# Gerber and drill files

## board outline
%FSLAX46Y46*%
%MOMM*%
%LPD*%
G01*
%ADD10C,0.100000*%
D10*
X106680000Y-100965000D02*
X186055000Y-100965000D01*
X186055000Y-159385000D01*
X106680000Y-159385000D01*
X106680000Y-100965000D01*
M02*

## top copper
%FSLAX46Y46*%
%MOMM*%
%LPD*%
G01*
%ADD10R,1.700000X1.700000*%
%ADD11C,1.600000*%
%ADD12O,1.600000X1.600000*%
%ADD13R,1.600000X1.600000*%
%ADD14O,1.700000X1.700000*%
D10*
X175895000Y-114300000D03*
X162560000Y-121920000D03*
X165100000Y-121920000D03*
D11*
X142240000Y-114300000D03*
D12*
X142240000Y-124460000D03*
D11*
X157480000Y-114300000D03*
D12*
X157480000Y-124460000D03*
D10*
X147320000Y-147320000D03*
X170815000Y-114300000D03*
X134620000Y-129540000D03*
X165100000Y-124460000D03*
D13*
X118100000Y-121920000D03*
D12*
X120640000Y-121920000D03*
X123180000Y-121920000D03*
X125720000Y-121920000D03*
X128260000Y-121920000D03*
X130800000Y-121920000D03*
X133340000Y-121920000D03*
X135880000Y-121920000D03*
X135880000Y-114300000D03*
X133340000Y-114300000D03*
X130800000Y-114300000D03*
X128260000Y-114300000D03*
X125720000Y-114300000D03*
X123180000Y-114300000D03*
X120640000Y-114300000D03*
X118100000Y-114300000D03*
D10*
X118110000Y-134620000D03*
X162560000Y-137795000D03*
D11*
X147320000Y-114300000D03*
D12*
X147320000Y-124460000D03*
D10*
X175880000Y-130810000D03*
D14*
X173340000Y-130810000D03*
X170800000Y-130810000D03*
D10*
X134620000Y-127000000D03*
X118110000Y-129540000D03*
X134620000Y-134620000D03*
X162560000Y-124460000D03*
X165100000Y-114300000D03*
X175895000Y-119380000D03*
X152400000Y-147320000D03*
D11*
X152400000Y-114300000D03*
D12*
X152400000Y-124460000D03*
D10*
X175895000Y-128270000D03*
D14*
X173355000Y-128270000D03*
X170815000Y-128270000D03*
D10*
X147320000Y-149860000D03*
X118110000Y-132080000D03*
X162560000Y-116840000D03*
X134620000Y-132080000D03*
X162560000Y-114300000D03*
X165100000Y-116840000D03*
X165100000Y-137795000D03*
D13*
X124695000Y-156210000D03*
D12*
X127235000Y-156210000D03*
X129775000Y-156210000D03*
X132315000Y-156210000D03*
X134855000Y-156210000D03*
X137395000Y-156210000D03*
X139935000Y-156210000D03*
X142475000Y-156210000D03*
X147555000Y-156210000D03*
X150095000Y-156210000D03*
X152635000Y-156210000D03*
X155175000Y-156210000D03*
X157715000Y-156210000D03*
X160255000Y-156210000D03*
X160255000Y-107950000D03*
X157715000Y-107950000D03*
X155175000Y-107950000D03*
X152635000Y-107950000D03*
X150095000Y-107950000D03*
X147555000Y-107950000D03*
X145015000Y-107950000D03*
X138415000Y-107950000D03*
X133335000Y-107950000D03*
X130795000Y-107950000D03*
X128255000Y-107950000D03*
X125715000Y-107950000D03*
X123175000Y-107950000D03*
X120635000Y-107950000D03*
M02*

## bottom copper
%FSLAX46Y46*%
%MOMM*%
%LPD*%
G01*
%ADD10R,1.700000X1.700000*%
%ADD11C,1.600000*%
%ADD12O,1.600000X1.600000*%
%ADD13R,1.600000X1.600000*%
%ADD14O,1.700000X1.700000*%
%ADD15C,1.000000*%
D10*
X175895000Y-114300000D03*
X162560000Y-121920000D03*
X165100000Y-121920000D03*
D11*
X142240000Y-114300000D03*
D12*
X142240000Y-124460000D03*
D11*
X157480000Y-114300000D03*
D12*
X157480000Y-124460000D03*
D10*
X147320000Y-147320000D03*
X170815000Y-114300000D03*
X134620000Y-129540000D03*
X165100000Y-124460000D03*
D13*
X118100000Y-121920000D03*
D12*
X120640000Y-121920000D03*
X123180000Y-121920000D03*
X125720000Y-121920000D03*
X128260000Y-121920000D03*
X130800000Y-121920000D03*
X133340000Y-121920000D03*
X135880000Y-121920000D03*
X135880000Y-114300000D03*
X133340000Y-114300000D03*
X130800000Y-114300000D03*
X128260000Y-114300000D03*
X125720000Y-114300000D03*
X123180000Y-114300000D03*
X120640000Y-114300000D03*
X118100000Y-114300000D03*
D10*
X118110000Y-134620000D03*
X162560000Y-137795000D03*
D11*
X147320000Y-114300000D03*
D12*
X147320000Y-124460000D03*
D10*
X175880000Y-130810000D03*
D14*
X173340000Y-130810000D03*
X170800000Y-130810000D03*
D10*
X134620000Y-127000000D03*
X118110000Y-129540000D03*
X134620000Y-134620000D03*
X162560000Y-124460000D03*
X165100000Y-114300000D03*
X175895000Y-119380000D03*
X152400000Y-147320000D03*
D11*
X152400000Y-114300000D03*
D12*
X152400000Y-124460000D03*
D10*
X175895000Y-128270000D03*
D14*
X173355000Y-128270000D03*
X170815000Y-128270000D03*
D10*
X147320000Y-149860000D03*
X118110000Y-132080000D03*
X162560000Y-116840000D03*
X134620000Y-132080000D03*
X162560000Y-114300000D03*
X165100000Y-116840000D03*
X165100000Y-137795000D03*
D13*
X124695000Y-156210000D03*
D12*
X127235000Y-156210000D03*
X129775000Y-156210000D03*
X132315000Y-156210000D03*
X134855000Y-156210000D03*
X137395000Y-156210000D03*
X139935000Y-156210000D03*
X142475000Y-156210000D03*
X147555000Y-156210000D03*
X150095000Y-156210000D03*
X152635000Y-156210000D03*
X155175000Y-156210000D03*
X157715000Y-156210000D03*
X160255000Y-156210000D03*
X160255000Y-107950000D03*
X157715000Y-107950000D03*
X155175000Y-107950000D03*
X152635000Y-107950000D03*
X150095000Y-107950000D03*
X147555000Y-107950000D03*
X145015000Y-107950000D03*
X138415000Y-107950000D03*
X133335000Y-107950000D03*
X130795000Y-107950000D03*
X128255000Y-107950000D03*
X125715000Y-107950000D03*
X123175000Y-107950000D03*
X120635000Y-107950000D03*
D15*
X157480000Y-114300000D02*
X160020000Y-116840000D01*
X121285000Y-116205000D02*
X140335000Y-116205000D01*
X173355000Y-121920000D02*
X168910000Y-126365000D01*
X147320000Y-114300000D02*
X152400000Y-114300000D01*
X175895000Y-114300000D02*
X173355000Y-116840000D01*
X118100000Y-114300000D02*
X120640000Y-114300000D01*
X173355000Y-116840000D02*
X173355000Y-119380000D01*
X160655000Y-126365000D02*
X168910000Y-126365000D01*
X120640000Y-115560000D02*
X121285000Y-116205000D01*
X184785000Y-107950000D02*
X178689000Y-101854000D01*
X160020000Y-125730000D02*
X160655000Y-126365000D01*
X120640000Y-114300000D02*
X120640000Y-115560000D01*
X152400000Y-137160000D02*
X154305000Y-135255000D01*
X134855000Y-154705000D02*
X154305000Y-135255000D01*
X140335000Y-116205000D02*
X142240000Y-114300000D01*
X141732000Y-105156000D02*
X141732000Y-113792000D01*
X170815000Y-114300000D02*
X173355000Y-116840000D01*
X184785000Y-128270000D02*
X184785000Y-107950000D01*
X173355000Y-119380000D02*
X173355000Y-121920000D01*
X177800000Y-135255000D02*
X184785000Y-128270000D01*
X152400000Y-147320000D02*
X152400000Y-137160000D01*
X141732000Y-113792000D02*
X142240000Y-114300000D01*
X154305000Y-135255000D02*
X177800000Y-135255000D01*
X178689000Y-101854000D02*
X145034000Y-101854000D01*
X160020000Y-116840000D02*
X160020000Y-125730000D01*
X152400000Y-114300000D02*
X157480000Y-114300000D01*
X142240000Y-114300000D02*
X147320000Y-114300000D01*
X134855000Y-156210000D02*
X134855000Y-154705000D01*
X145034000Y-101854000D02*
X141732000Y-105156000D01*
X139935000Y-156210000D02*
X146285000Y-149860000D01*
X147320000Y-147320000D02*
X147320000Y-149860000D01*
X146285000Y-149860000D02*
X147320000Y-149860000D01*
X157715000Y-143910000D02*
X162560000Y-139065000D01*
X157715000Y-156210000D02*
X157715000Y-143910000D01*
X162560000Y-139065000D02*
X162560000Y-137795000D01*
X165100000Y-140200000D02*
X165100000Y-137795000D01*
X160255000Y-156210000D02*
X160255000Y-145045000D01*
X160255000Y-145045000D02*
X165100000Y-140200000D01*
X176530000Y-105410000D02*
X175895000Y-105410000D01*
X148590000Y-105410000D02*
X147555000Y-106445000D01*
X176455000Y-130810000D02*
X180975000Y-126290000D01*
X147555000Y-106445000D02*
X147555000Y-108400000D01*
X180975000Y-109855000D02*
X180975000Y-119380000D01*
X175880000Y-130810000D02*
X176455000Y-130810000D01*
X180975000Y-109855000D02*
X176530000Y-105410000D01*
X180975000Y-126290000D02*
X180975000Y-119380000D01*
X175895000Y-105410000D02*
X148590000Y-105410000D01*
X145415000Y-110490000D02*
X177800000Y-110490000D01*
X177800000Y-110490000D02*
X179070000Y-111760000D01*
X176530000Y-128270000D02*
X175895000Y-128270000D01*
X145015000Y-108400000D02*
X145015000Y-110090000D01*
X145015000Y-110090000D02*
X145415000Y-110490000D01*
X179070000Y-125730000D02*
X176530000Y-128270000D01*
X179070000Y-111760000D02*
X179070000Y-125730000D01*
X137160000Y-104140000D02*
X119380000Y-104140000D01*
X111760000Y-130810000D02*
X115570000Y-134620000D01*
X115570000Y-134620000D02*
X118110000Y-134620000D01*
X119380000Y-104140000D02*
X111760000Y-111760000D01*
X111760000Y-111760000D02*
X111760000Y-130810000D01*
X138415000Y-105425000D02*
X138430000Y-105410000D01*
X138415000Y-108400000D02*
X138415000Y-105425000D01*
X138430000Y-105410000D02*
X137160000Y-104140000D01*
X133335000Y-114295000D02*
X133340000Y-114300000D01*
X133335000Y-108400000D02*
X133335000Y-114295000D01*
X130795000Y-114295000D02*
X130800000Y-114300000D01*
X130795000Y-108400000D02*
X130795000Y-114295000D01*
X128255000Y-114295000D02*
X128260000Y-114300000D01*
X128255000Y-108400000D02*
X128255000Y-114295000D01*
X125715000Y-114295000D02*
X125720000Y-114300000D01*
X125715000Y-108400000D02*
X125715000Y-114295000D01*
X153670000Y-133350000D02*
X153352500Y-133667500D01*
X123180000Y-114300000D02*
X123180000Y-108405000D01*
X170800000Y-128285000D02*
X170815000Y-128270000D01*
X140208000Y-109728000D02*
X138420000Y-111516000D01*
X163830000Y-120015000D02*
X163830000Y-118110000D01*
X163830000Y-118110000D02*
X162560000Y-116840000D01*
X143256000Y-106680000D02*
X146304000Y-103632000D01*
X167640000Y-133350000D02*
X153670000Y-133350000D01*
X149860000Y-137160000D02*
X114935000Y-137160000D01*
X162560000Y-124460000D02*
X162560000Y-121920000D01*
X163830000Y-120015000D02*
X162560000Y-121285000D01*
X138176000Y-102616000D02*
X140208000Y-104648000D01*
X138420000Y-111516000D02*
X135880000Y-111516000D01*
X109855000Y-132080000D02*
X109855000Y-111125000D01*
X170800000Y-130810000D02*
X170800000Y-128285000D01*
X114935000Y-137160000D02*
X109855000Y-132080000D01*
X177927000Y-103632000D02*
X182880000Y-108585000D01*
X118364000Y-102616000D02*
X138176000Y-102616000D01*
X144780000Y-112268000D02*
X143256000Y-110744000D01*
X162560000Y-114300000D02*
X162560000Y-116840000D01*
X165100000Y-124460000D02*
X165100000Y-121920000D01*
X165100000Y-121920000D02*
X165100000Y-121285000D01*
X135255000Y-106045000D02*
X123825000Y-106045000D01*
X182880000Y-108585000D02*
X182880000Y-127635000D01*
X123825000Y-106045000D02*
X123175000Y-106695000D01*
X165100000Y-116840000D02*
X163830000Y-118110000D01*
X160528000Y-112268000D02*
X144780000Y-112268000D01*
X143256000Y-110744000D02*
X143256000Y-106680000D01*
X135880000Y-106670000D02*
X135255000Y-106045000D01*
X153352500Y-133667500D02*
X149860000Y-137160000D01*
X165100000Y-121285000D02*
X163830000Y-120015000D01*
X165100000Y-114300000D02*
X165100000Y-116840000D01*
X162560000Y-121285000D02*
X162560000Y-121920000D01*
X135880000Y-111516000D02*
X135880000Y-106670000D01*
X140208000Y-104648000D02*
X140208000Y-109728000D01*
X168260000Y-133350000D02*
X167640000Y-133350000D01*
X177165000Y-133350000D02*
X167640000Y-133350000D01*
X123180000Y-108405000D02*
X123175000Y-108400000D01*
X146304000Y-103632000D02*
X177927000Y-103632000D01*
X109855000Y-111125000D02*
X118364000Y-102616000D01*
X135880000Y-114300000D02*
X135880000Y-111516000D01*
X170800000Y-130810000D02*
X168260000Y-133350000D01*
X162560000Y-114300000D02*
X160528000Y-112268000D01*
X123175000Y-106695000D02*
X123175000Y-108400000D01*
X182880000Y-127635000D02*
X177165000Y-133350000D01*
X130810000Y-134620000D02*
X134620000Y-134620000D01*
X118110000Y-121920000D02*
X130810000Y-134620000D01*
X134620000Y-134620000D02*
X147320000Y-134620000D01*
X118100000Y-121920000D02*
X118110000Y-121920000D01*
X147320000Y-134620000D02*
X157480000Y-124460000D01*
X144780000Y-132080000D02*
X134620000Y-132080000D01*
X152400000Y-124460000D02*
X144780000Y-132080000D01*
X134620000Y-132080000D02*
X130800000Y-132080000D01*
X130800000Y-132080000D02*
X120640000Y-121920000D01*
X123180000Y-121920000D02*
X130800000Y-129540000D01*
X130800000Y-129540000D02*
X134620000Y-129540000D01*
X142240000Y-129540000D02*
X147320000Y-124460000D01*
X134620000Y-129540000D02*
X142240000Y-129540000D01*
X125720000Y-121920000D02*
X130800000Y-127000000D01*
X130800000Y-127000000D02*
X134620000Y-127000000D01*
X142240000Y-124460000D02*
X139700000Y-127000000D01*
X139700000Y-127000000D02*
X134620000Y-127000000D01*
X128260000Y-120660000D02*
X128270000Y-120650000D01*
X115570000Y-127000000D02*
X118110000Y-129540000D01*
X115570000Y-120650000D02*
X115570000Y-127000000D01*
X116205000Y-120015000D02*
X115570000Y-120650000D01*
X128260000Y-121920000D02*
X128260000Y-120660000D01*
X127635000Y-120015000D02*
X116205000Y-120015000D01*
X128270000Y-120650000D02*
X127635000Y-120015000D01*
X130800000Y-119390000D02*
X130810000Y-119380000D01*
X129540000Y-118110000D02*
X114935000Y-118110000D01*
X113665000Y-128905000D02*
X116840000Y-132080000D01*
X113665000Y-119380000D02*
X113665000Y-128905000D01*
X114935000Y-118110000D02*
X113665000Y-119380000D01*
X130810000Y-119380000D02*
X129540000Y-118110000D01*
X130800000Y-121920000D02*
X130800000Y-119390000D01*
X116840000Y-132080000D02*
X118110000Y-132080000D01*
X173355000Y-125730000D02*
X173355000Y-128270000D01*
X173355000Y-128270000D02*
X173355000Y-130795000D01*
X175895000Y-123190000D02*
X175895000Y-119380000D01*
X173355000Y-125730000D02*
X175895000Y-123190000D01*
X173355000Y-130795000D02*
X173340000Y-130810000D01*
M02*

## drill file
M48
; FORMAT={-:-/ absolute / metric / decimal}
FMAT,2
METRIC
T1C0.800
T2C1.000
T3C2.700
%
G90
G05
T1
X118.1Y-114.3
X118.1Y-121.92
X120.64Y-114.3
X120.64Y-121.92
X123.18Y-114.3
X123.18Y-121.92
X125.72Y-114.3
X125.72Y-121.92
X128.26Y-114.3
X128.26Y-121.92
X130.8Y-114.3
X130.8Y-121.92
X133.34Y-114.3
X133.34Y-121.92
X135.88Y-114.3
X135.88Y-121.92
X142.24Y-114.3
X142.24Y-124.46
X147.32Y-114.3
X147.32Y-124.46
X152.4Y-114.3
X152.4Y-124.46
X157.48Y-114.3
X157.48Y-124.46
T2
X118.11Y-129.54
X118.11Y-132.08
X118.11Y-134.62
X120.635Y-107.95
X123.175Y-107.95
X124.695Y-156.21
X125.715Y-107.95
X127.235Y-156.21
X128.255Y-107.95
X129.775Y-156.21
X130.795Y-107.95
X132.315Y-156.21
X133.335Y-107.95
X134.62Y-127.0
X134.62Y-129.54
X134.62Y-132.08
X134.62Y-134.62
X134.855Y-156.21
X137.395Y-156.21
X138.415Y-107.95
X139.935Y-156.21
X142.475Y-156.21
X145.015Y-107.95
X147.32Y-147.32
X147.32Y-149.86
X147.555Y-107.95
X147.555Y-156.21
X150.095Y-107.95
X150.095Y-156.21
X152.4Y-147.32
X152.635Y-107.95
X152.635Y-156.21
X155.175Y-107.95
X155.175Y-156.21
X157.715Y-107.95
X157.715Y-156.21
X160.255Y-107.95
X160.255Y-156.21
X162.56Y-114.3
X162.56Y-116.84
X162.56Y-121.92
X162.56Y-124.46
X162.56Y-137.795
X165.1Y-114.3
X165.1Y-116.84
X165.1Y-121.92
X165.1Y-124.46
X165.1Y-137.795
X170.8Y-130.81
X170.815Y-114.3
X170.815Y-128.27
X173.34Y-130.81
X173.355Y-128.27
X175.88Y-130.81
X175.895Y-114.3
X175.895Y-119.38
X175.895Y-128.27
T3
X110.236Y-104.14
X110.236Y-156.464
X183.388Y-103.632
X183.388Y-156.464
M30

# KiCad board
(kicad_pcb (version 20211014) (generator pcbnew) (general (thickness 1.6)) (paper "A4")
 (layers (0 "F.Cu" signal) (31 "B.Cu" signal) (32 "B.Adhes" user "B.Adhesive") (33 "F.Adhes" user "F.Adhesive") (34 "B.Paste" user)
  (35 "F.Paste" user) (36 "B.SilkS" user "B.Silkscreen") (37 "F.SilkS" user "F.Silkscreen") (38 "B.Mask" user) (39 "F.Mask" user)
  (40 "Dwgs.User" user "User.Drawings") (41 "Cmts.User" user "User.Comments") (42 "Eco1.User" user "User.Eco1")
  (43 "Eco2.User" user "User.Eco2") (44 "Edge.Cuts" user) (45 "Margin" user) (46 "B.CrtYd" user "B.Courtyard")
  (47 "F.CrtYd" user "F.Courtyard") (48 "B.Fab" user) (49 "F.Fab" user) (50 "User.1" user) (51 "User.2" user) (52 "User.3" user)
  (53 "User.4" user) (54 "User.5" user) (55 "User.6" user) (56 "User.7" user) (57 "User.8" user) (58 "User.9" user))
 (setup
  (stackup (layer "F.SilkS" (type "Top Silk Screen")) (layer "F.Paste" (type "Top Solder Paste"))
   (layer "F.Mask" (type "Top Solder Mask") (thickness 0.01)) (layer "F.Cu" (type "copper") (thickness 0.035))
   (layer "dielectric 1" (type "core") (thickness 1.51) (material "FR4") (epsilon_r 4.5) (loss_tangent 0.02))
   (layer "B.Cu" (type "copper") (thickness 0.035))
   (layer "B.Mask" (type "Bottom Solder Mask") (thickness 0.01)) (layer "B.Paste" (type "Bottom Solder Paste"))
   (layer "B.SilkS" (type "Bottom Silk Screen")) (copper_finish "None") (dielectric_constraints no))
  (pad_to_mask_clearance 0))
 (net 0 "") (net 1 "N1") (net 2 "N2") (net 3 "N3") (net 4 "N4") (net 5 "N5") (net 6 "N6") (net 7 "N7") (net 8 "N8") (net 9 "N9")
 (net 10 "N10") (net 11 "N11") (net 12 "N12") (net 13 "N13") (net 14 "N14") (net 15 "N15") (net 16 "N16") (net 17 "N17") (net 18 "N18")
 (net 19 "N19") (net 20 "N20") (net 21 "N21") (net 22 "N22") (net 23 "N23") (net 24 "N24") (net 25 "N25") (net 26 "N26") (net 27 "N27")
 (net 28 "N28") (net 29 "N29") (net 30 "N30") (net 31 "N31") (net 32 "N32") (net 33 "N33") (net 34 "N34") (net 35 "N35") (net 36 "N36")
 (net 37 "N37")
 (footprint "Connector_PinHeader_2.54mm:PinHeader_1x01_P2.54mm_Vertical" (layer "F.Cu") (at 175.895 114.3)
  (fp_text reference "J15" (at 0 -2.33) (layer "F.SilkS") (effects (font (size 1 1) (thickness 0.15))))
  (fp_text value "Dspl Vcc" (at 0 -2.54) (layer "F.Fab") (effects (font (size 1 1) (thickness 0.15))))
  (pad "1" thru_hole rect (at 0 0) (size 1.7 1.7) (drill 1) (layers *.Cu *.Mask) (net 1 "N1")))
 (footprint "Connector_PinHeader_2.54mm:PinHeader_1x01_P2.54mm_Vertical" (layer "F.Cu") (at 162.56 121.92)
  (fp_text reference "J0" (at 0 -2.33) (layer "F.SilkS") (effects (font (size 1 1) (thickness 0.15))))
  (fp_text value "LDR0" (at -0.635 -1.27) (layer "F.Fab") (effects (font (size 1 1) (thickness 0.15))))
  (pad "1" thru_hole rect (at 0 0) (size 1.7 1.7) (drill 1) (layers *.Cu *.Mask) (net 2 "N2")))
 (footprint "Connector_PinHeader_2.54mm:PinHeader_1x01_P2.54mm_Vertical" (layer "F.Cu") (at 165.1 121.92)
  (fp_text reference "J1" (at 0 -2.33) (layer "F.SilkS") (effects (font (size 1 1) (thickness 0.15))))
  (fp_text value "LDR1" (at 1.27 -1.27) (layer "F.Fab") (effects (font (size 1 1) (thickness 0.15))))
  (pad "1" thru_hole rect (at 0 0) (size 1.7 1.7) (drill 1) (layers *.Cu *.Mask) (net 2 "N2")))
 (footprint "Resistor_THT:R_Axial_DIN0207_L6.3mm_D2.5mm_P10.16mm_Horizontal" (layer "F.Cu") (at 142.24 114.3 -90)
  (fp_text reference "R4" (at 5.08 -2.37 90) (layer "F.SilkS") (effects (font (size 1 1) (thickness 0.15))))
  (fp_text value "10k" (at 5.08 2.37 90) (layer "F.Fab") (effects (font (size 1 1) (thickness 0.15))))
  (pad "1" thru_hole circle (at 0 0 270) (size 1.6 1.6) (drill 0.8) (layers *.Cu *.Mask) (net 1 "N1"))
  (pad "2" thru_hole oval (at 10.16 0 270) (size 1.6 1.6) (drill 0.8) (layers *.Cu *.Mask) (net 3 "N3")))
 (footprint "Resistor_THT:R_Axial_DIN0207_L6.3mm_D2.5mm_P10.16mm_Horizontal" (layer "F.Cu") (at 157.48 114.3 -90)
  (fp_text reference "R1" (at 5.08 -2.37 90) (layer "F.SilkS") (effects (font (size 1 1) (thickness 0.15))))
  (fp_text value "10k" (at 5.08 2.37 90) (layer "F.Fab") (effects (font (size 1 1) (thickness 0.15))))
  (pad "1" thru_hole circle (at 0 0 270) (size 1.6 1.6) (drill 0.8) (layers *.Cu *.Mask) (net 1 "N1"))
  (pad "2" thru_hole oval (at 10.16 0 270) (size 1.6 1.6) (drill 0.8) (layers *.Cu *.Mask) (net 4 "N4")))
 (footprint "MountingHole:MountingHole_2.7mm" (layer "F.Cu") (at 110.236 156.464)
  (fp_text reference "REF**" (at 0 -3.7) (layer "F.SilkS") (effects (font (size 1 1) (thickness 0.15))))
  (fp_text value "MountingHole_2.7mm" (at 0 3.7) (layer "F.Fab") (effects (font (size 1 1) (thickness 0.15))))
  (pad "" np_thru_hole circle (at 0 0) (size 2.7 2.7) (drill 2.7) (layers *.Cu *.Mask)))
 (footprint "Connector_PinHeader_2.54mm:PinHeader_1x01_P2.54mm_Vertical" (layer "F.Cu") (at 147.32 147.32)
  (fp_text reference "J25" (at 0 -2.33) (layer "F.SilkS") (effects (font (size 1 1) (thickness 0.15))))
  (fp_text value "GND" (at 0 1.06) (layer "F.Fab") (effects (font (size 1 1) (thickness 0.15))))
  (pad "1" thru_hole rect (at 0 0) (size 1.7 1.7) (drill 1) (layers *.Cu *.Mask) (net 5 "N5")))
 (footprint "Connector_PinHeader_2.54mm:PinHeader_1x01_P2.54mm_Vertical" (layer "F.Cu") (at 170.815 114.3)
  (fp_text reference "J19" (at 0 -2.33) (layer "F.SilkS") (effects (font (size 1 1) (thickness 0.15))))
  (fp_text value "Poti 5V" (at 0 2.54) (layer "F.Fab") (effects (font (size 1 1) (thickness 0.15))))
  (pad "1" thru_hole rect (at 0 0) (size 1.7 1.7) (drill 1) (layers *.Cu *.Mask) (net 1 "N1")))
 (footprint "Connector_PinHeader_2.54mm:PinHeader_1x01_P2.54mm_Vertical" (layer "F.Cu") (at 134.62 129.54 90)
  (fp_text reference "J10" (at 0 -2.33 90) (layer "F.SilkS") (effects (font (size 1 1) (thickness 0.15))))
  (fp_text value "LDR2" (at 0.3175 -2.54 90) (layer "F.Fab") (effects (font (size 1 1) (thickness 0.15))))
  (pad "1" thru_hole rect (at 0 0 90) (size 1.7 1.7) (drill 1) (layers *.Cu *.Mask) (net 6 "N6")))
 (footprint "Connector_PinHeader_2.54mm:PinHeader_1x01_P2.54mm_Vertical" (layer "F.Cu") (at 165.1 124.46)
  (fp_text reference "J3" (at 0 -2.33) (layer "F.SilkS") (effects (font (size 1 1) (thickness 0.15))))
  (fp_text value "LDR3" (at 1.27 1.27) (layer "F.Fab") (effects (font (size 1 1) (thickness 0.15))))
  (pad "1" thru_hole rect (at 0 0) (size 1.7 1.7) (drill 1) (layers *.Cu *.Mask) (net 2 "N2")))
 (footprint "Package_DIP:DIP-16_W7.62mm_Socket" (layer "F.Cu") (at 118.1 121.92 90)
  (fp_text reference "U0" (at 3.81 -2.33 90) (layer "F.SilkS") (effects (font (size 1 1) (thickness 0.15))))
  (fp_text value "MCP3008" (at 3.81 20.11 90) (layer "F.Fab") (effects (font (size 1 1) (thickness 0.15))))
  (pad "1" thru_hole rect (at 0 0 90) (size 1.6 1.6) (drill 0.8) (layers *.Cu *.Mask) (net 4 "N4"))
  (pad "2" thru_hole oval (at 0 2.54 90) (size 1.6 1.6) (drill 0.8) (layers *.Cu *.Mask) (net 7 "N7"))
  (pad "3" thru_hole oval (at 0 5.08 90) (size 1.6 1.6) (drill 0.8) (layers *.Cu *.Mask) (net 6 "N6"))
  (pad "4" thru_hole oval (at 0 7.62 90) (size 1.6 1.6) (drill 0.8) (layers *.Cu *.Mask) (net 3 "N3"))
  (pad "5" thru_hole oval (at 0 10.16 90) (size 1.6 1.6) (drill 0.8) (layers *.Cu *.Mask) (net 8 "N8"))
  (pad "6" thru_hole oval (at 0 12.7 90) (size 1.6 1.6) (drill 0.8) (layers *.Cu *.Mask) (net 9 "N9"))
  (pad "7" thru_hole oval (at 0 15.24 90) (size 1.6 1.6) (drill 0.8) (layers *.Cu *.Mask) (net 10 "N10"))
  (pad "8" thru_hole oval (at 0 17.78 90) (size 1.6 1.6) (drill 0.8) (layers *.Cu *.Mask) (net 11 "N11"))
  (pad "9" thru_hole oval (at 7.62 17.78 90) (size 1.6 1.6) (drill 0.8) (layers *.Cu *.Mask) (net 2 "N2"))
  (pad "10" thru_hole oval (at 7.62 15.24 90) (size 1.6 1.6) (drill 0.8) (layers *.Cu *.Mask) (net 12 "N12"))
  (pad "11" thru_hole oval (at 7.62 12.7 90) (size 1.6 1.6) (drill 0.8) (layers *.Cu *.Mask) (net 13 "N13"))
  (pad "12" thru_hole oval (at 7.62 10.16 90) (size 1.6 1.6) (drill 0.8) (layers *.Cu *.Mask) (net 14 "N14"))
  (pad "13" thru_hole oval (at 7.62 7.62 90) (size 1.6 1.6) (drill 0.8) (layers *.Cu *.Mask) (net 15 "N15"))
  (pad "14" thru_hole oval (at 7.62 5.08 90) (size 1.6 1.6) (drill 0.8) (layers *.Cu *.Mask) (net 2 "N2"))
  (pad "15" thru_hole oval (at 7.62 2.54 90) (size 1.6 1.6) (drill 0.8) (layers *.Cu *.Mask) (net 1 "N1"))
  (pad "16" thru_hole oval (at 7.62 0 90) (size 1.6 1.6) (drill 0.8) (layers *.Cu *.Mask) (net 1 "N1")))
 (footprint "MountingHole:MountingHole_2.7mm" (layer "F.Cu") (at 183.388 156.464)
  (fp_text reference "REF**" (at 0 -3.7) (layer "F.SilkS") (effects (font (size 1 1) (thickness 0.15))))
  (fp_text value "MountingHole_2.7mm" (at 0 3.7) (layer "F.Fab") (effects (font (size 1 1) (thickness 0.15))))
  (pad "" np_thru_hole circle (at 0 0) (size 2.7 2.7) (drill 2.7) (layers *.Cu *.Mask)))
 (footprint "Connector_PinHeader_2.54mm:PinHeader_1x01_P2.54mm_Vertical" (layer "F.Cu") (at 118.11 134.62 -90)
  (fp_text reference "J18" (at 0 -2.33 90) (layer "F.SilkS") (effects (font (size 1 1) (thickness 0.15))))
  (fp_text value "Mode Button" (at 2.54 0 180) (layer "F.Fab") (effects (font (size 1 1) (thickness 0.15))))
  (pad "1" thru_hole rect (at 0 0 270) (size 1.7 1.7) (drill 1) (layers *.Cu *.Mask) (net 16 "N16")))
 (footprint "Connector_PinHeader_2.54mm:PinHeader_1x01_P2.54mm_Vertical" (layer "F.Cu") (at 162.56 137.795)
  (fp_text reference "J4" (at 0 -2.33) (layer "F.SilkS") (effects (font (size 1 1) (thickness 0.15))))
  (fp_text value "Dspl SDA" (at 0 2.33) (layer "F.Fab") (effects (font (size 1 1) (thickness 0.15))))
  (pad "1" thru_hole rect (at 0 0) (size 1.7 1.7) (drill 1) (layers *.Cu *.Mask) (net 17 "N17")))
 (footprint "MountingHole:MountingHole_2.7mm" (layer "F.Cu") (at 110.236 104.14)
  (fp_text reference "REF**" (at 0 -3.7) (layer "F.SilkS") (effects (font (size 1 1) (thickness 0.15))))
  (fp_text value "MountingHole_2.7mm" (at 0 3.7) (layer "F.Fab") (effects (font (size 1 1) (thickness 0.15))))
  (pad "" np_thru_hole circle (at 0 0) (size 2.7 2.7) (drill 2.7) (layers *.Cu *.Mask)))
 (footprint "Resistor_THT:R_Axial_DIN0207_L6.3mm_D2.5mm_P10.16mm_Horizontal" (layer "F.Cu") (at 147.32 114.3 -90)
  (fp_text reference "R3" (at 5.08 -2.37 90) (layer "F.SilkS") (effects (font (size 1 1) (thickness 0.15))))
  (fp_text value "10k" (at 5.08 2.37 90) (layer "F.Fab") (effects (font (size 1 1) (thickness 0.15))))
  (pad "1" thru_hole circle (at 0 0 270) (size 1.6 1.6) (drill 0.8) (layers *.Cu *.Mask) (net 1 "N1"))
  (pad "2" thru_hole oval (at 10.16 0 270) (size 1.6 1.6) (drill 0.8) (layers *.Cu *.Mask) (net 6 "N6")))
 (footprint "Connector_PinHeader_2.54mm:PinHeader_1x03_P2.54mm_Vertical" (layer "F.Cu") (at 175.88 130.81 -90)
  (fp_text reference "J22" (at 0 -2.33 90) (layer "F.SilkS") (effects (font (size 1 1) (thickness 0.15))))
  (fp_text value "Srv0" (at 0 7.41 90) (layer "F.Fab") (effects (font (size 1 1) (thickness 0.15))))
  (pad "1" thru_hole rect (at 0 0 270) (size 1.7 1.7) (drill 1) (layers *.Cu *.Mask) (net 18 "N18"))
  (pad "2" thru_hole oval (at 0 2.54 270) (size 1.7 1.7) (drill 1) (layers *.Cu *.Mask) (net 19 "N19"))
  (pad "3" thru_hole oval (at 0 5.08 270) (size 1.7 1.7) (drill 1) (layers *.Cu *.Mask) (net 2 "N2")))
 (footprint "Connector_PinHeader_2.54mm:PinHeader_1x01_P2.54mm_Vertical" (layer "F.Cu") (at 134.62 127)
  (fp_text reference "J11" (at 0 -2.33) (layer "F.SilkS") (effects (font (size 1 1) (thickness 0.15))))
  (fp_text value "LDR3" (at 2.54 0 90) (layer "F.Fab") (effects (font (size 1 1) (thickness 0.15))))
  (pad "1" thru_hole rect (at 0 0) (size 1.7 1.7) (drill 1) (layers *.Cu *.Mask) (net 3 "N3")))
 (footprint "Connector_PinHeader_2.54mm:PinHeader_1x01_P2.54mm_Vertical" (layer "F.Cu") (at 118.11 129.54 -90)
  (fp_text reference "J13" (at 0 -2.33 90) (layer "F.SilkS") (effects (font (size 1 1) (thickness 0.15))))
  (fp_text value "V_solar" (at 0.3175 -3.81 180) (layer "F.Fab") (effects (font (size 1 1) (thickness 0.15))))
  (pad "1" thru_hole rect (at 0 0 270) (size 1.7 1.7) (drill 1) (layers *.Cu *.Mask) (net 8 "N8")))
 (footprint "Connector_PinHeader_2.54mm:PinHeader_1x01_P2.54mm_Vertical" (layer "F.Cu") (at 134.62 134.62 90)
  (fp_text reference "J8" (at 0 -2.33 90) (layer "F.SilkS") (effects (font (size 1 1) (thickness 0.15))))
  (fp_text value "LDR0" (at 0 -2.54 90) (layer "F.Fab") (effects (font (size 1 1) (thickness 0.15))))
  (pad "1" thru_hole rect (at 0 0 90) (size 1.7 1.7) (drill 1) (layers *.Cu *.Mask) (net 4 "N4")))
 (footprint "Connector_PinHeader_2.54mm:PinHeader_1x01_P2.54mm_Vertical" (layer "F.Cu") (at 162.56 124.46)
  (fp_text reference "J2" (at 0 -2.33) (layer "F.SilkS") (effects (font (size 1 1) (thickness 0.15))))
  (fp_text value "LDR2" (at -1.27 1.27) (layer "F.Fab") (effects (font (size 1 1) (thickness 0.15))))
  (pad "1" thru_hole rect (at 0 0) (size 1.7 1.7) (drill 1) (layers *.Cu *.Mask) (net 2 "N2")))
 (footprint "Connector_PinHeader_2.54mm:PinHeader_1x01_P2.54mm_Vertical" (layer "F.Cu") (at 165.1 114.3)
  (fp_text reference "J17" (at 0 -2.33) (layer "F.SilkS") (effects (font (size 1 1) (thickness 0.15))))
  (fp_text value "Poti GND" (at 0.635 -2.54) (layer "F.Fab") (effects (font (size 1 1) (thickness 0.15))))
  (pad "1" thru_hole rect (at 0 0) (size 1.7 1.7) (drill 1) (layers *.Cu *.Mask) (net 2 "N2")))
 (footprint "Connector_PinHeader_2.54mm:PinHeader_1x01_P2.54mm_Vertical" (layer "F.Cu") (at 175.895 119.38)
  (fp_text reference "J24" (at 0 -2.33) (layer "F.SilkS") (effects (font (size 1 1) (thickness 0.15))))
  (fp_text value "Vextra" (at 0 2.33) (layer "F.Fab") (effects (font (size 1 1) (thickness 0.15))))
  (pad "1" thru_hole rect (at 0 0) (size 1.7 1.7) (drill 1) (layers *.Cu *.Mask) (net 19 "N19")))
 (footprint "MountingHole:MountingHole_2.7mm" (layer "F.Cu") (at 183.388 103.632)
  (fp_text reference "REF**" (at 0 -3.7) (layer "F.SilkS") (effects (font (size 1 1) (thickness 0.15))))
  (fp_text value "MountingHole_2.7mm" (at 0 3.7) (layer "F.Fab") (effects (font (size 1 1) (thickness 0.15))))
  (pad "" np_thru_hole circle (at 0 0) (size 2.7 2.7) (drill 2.7) (layers *.Cu *.Mask)))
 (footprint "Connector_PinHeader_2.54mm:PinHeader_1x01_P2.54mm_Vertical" (layer "F.Cu") (at 152.4 147.32)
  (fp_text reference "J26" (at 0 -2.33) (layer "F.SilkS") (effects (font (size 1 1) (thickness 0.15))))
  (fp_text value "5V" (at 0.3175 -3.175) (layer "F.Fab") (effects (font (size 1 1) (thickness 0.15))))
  (pad "1" thru_hole rect (at 0 0) (size 1.7 1.7) (drill 1) (layers *.Cu *.Mask) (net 1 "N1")))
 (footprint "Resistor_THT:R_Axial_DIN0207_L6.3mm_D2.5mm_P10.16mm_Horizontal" (layer "F.Cu") (at 152.4 114.3 -90)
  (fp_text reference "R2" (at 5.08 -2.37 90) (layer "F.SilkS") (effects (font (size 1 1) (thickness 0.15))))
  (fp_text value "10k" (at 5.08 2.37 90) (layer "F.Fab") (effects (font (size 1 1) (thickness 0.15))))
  (pad "1" thru_hole circle (at 0 0 270) (size 1.6 1.6) (drill 0.8) (layers *.Cu *.Mask) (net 1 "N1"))
  (pad "2" thru_hole oval (at 10.16 0 270) (size 1.6 1.6) (drill 0.8) (layers *.Cu *.Mask) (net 7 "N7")))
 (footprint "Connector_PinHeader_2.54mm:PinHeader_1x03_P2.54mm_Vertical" (layer "F.Cu") (at 175.895 128.27 -90)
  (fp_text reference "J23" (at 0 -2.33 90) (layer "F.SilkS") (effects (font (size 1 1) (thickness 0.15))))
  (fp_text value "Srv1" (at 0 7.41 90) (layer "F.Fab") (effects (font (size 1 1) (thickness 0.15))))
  (pad "1" thru_hole rect (at 0 0 270) (size 1.7 1.7) (drill 1) (layers *.Cu *.Mask) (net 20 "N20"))
  (pad "2" thru_hole oval (at 0 2.54 270) (size 1.7 1.7) (drill 1) (layers *.Cu *.Mask) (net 19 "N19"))
  (pad "3" thru_hole oval (at 0 5.08 270) (size 1.7 1.7) (drill 1) (layers *.Cu *.Mask) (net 2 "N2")))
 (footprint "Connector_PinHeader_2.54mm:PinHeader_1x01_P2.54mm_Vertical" (layer "F.Cu") (at 147.32 149.86)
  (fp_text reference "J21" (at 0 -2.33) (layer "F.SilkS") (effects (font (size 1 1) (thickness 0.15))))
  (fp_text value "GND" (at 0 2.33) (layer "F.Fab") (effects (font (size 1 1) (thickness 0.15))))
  (pad "1" thru_hole rect (at 0 0) (size 1.7 1.7) (drill 1) (layers *.Cu *.Mask) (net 5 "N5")))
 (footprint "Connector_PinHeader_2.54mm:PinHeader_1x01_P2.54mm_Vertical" (layer "F.Cu") (at 118.11 132.08 -90)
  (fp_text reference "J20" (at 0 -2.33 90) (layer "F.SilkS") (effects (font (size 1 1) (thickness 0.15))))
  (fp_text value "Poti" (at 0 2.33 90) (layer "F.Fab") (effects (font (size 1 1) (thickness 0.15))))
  (pad "1" thru_hole rect (at 0 0 270) (size 1.7 1.7) (drill 1) (layers *.Cu *.Mask) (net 9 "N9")))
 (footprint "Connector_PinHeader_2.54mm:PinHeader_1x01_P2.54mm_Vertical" (layer "F.Cu") (at 162.56 116.84)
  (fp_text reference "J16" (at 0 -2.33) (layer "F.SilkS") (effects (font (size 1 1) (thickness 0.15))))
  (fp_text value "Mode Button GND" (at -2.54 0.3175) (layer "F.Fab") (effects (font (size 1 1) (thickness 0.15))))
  (pad "1" thru_hole rect (at 0 0) (size 1.7 1.7) (drill 1) (layers *.Cu *.Mask) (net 2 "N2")))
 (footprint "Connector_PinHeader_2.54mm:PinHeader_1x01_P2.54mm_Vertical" (layer "F.Cu") (at 134.62 132.08 90)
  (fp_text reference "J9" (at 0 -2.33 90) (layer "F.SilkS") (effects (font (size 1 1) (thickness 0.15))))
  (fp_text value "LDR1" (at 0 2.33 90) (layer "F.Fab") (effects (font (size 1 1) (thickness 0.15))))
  (pad "1" thru_hole rect (at 0 0 90) (size 1.7 1.7) (drill 1) (layers *.Cu *.Mask) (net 7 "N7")))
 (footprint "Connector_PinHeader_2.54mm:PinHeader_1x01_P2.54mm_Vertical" (layer "F.Cu") (at 162.56 114.3)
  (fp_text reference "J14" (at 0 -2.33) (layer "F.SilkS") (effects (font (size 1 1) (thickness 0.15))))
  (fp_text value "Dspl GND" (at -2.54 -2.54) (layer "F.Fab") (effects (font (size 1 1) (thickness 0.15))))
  (pad "1" thru_hole rect (at 0 0) (size 1.7 1.7) (drill 1) (layers *.Cu *.Mask) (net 2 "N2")))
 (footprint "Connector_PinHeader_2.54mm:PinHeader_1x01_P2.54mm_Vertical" (layer "F.Cu") (at 165.1 116.84)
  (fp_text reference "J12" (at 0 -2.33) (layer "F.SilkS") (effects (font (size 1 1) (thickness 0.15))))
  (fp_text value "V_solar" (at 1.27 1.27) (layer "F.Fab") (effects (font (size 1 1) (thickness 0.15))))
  (pad "1" thru_hole rect (at 0 0) (size 1.7 1.7) (drill 1) (layers *.Cu *.Mask) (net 2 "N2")))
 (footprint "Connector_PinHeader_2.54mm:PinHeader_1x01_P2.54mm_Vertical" (layer "F.Cu") (at 165.1 137.795)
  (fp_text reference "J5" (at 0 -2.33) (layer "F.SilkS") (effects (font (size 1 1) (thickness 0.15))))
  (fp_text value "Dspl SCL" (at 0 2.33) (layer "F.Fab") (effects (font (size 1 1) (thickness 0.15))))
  (pad "1" thru_hole rect (at 0 0) (size 1.7 1.7) (drill 1) (layers *.Cu *.Mask) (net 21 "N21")))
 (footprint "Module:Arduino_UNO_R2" (layer "B.Cu") (at 124.695 156.21)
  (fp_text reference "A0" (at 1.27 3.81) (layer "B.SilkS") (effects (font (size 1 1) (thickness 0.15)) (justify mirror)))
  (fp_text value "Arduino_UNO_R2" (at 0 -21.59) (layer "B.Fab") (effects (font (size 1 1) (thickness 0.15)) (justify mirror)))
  (pad "1" thru_hole rect (at 0 0 270) (size 1.6 1.6) (drill 1) (layers *.Cu *.Mask) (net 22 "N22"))
  (pad "2" thru_hole oval (at 2.54 0 270) (size 1.6 1.6) (drill 1) (layers *.Cu *.Mask) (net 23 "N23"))
  (pad "3" thru_hole oval (at 5.08 0 270) (size 1.6 1.6) (drill 1) (layers *.Cu *.Mask) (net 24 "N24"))
  (pad "4" thru_hole oval (at 7.62 0 270) (size 1.6 1.6) (drill 1) (layers *.Cu *.Mask) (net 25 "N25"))
  (pad "5" thru_hole oval (at 10.16 0 270) (size 1.6 1.6) (drill 1) (layers *.Cu *.Mask) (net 1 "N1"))
  (pad "6" thru_hole oval (at 12.7 0 270) (size 1.6 1.6) (drill 1) (layers *.Cu *.Mask) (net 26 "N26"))
  (pad "7" thru_hole oval (at 15.24 0 270) (size 1.6 1.6) (drill 1) (layers *.Cu *.Mask) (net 5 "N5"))
  (pad "8" thru_hole oval (at 17.78 0 270) (size 1.6 1.6) (drill 1) (layers *.Cu *.Mask) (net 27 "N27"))
  (pad "9" thru_hole oval (at 22.86 0 270) (size 1.6 1.6) (drill 1) (layers *.Cu *.Mask) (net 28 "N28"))
  (pad "10" thru_hole oval (at 25.4 0 270) (size 1.6 1.6) (drill 1) (layers *.Cu *.Mask) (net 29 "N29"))
  (pad "11" thru_hole oval (at 27.94 0 270) (size 1.6 1.6) (drill 1) (layers *.Cu *.Mask) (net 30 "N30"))
  (pad "12" thru_hole oval (at 30.48 0 270) (size 1.6 1.6) (drill 1) (layers *.Cu *.Mask) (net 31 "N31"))
  (pad "13" thru_hole oval (at 33.02 0 270) (size 1.6 1.6) (drill 1) (layers *.Cu *.Mask) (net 17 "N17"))
  (pad "14" thru_hole oval (at 35.56 0 270) (size 1.6 1.6) (drill 1) (layers *.Cu *.Mask) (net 21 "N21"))
  (pad "15" thru_hole oval (at 35.56 -48.26 270) (size 1.6 1.6) (drill 1) (layers *.Cu *.Mask) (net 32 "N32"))
  (pad "16" thru_hole oval (at 33.02 -48.26 270) (size 1.6 1.6) (drill 1) (layers *.Cu *.Mask) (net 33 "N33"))
  (pad "17" thru_hole oval (at 30.48 -48.26 270) (size 1.6 1.6) (drill 1) (layers *.Cu *.Mask) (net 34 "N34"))
  (pad "18" thru_hole oval (at 27.94 -48.26 270) (size 1.6 1.6) (drill 1) (layers *.Cu *.Mask) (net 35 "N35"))
  (pad "19" thru_hole oval (at 25.4 -48.26 270) (size 1.6 1.6) (drill 1) (layers *.Cu *.Mask) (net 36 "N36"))
  (pad "20" thru_hole oval (at 22.86 -48.26 270) (size 1.6 1.6) (drill 1) (layers *.Cu *.Mask) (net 18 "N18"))
  (pad "21" thru_hole oval (at 20.32 -48.26 270) (size 1.6 1.6) (drill 1) (layers *.Cu *.Mask) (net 20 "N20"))
  (pad "23" thru_hole oval (at 13.72 -48.26 270) (size 1.6 1.6) (drill 1) (layers *.Cu *.Mask) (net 16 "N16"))
  (pad "25" thru_hole oval (at 8.64 -48.26 270) (size 1.6 1.6) (drill 1) (layers *.Cu *.Mask) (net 12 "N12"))
  (pad "26" thru_hole oval (at 6.1 -48.26 270) (size 1.6 1.6) (drill 1) (layers *.Cu *.Mask) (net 13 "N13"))
  (pad "27" thru_hole oval (at 3.56 -48.26 270) (size 1.6 1.6) (drill 1) (layers *.Cu *.Mask) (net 14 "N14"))
  (pad "28" thru_hole oval (at 1.02 -48.26 270) (size 1.6 1.6) (drill 1) (layers *.Cu *.Mask) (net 15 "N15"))
  (pad "29" thru_hole oval (at -1.52 -48.26 270) (size 1.6 1.6) (drill 1) (layers *.Cu *.Mask) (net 2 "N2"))
  (pad "30" thru_hole oval (at -4.06 -48.26 270) (size 1.6 1.6) (drill 1) (layers *.Cu *.Mask) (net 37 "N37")))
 (gr_rect (start 106.68 159.385) (end 186.055 100.965) (layer "Edge.Cuts") (width 0.1) (fill none))
 (segment (start 157.48 114.3) (end 160.02 116.84) (width 1) (layer "B.Cu") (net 1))
 (segment (start 121.285 116.205) (end 140.335 116.205) (width 1) (layer "B.Cu") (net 1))
 (segment (start 173.355 121.92) (end 168.91 126.365) (width 1) (layer "B.Cu") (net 1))
 (segment (start 147.32 114.3) (end 152.4 114.3) (width 1) (layer "B.Cu") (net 1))
 (segment (start 175.895 114.3) (end 173.355 116.84) (width 1) (layer "B.Cu") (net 1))
 (segment (start 118.1 114.3) (end 120.64 114.3) (width 1) (layer "B.Cu") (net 1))
 (segment (start 173.355 116.84) (end 173.355 119.38) (width 1) (layer "B.Cu") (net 1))
 (segment (start 160.655 126.365) (end 168.91 126.365) (width 1) (layer "B.Cu") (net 1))
 (segment (start 120.64 115.56) (end 121.285 116.205) (width 1) (layer "B.Cu") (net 1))
 (segment (start 184.785 107.95) (end 178.689 101.854) (width 1) (layer "B.Cu") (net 1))
 (segment (start 160.02 125.73) (end 160.655 126.365) (width 1) (layer "B.Cu") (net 1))
 (segment (start 120.64 114.3) (end 120.64 115.56) (width 1) (layer "B.Cu") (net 1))
 (segment (start 152.4 137.16) (end 154.305 135.255) (width 1) (layer "B.Cu") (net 1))
 (segment (start 134.855 154.705) (end 154.305 135.255) (width 1) (layer "B.Cu") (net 1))
 (segment (start 140.335 116.205) (end 142.24 114.3) (width 1) (layer "B.Cu") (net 1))
 (segment (start 141.732 105.156) (end 141.732 113.792) (width 1) (layer "B.Cu") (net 1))
 (segment (start 170.815 114.3) (end 173.355 116.84) (width 1) (layer "B.Cu") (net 1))
 (segment (start 184.785 128.27) (end 184.785 107.95) (width 1) (layer "B.Cu") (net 1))
 (segment (start 173.355 119.38) (end 173.355 121.92) (width 1) (layer "B.Cu") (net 1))
 (segment (start 177.8 135.255) (end 184.785 128.27) (width 1) (layer "B.Cu") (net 1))
 (segment (start 152.4 147.32) (end 152.4 137.16) (width 1) (layer "B.Cu") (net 1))
 (segment (start 141.732 113.792) (end 142.24 114.3) (width 1) (layer "B.Cu") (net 1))
 (segment (start 154.305 135.255) (end 177.8 135.255) (width 1) (layer "B.Cu") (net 1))
 (segment (start 178.689 101.854) (end 145.034 101.854) (width 1) (layer "B.Cu") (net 1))
 (segment (start 160.02 116.84) (end 160.02 125.73) (width 1) (layer "B.Cu") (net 1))
 (segment (start 152.4 114.3) (end 157.48 114.3) (width 1) (layer "B.Cu") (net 1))
 (segment (start 142.24 114.3) (end 147.32 114.3) (width 1) (layer "B.Cu") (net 1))
 (segment (start 134.855 156.21) (end 134.855 154.705) (width 1) (layer "B.Cu") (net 1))
 (segment (start 145.034 101.854) (end 141.732 105.156) (width 1) (layer "B.Cu") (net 1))
 (segment (start 139.935 156.21) (end 146.285 149.86) (width 1) (layer "B.Cu") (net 5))
 (segment (start 147.32 147.32) (end 147.32 149.86) (width 1) (layer "B.Cu") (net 5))
 (segment (start 146.285 149.86) (end 147.32 149.86) (width 1) (layer "B.Cu") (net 5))
 (segment (start 157.715 143.91) (end 162.56 139.065) (width 1) (layer "B.Cu") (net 17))
 (segment (start 157.715 156.21) (end 157.715 143.91) (width 1) (layer "B.Cu") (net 17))
 (segment (start 162.56 139.065) (end 162.56 137.795) (width 1) (layer "B.Cu") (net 17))
 (segment (start 165.1 140.2) (end 165.1 137.795) (width 1) (layer "B.Cu") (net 21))
 (segment (start 160.255 156.21) (end 160.255 145.045) (width 1) (layer "B.Cu") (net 21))
 (segment (start 160.255 145.045) (end 165.1 140.2) (width 1) (layer "B.Cu") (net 21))
 (segment (start 176.53 105.41) (end 175.895 105.41) (width 1) (layer "B.Cu") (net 18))
 (segment (start 148.59 105.41) (end 147.555 106.445) (width 1) (layer "B.Cu") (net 18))
 (segment (start 176.455 130.81) (end 180.975 126.29) (width 1) (layer "B.Cu") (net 18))
 (segment (start 147.555 106.445) (end 147.555 108.4) (width 1) (layer "B.Cu") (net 18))
 (segment (start 180.975 109.855) (end 180.975 119.38) (width 1) (layer "B.Cu") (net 18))
 (segment (start 175.88 130.81) (end 176.455 130.81) (width 1) (layer "B.Cu") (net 18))
 (segment (start 180.975 109.855) (end 176.53 105.41) (width 1) (layer "B.Cu") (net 18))
 (segment (start 180.975 126.29) (end 180.975 119.38) (width 1) (layer "B.Cu") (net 18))
 (segment (start 175.895 105.41) (end 148.59 105.41) (width 1) (layer "B.Cu") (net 18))
 (segment (start 145.415 110.49) (end 177.8 110.49) (width 1) (layer "B.Cu") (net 20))
 (segment (start 177.8 110.49) (end 179.07 111.76) (width 1) (layer "B.Cu") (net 20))
 (segment (start 176.53 128.27) (end 175.895 128.27) (width 1) (layer "B.Cu") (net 20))
 (segment (start 145.015 108.4) (end 145.015 110.09) (width 1) (layer "B.Cu") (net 20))
 (segment (start 145.015 110.09) (end 145.415 110.49) (width 1) (layer "B.Cu") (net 20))
 (segment (start 179.07 125.73) (end 176.53 128.27) (width 1) (layer "B.Cu") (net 20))
 (segment (start 179.07 111.76) (end 179.07 125.73) (width 1) (layer "B.Cu") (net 20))
 (segment (start 137.16 104.14) (end 119.38 104.14) (width 1) (layer "B.Cu") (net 16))
 (segment (start 111.76 130.81) (end 115.57 134.62) (width 1) (layer "B.Cu") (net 16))
 (segment (start 115.57 134.62) (end 118.11 134.62) (width 1) (layer "B.Cu") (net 16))
 (segment (start 119.38 104.14) (end 111.76 111.76) (width 1) (layer "B.Cu") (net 16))
 (segment (start 111.76 111.76) (end 111.76 130.81) (width 1) (layer "B.Cu") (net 16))
 (segment (start 138.415 105.425) (end 138.43 105.41) (width 1) (layer "B.Cu") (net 16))
 (segment (start 138.415 108.4) (end 138.415 105.425) (width 1) (layer "B.Cu") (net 16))
 (segment (start 138.43 105.41) (end 137.16 104.14) (width 1) (layer "B.Cu") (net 16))
 (segment (start 133.335 114.295) (end 133.34 114.3) (width 1) (layer "B.Cu") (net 12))
 (segment (start 133.335 108.4) (end 133.335 114.295) (width 1) (layer "B.Cu") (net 12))
 (segment (start 130.795 114.295) (end 130.8 114.3) (width 1) (layer "B.Cu") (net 13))
 (segment (start 130.795 108.4) (end 130.795 114.295) (width 1) (layer "B.Cu") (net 13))
 (segment (start 128.255 114.295) (end 128.26 114.3) (width 1) (layer "B.Cu") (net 14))
 (segment (start 128.255 108.4) (end 128.255 114.295) (width 1) (layer "B.Cu") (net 14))
 (segment (start 125.715 114.295) (end 125.72 114.3) (width 1) (layer "B.Cu") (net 15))
 (segment (start 125.715 108.4) (end 125.715 114.295) (width 1) (layer "B.Cu") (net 15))
 (segment (start 153.67 133.35) (end 153.3525 133.6675) (width 1) (layer "B.Cu") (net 2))
 (segment (start 123.18 114.3) (end 123.18 108.405) (width 1) (layer "B.Cu") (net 2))
 (segment (start 170.8 128.285) (end 170.815 128.27) (width 1) (layer "B.Cu") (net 2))
 (segment (start 140.208 109.728) (end 138.42 111.516) (width 1) (layer "B.Cu") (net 2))
 (segment (start 163.83 120.015) (end 163.83 118.11) (width 1) (layer "B.Cu") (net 2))
 (segment (start 163.83 118.11) (end 162.56 116.84) (width 1) (layer "B.Cu") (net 2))
 (segment (start 143.256 106.68) (end 146.304 103.632) (width 1) (layer "B.Cu") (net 2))
 (segment (start 167.64 133.35) (end 153.67 133.35) (width 1) (layer "B.Cu") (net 2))
 (segment (start 149.86 137.16) (end 114.935 137.16) (width 1) (layer "B.Cu") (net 2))
 (segment (start 162.56 124.46) (end 162.56 121.92) (width 1) (layer "B.Cu") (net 2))
 (segment (start 163.83 120.015) (end 162.56 121.285) (width 1) (layer "B.Cu") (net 2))
 (segment (start 138.176 102.616) (end 140.208 104.648) (width 1) (layer "B.Cu") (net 2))
 (segment (start 138.42 111.516) (end 135.88 111.516) (width 1) (layer "B.Cu") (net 2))
 (segment (start 109.855 132.08) (end 109.855 111.125) (width 1) (layer "B.Cu") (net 2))
 (segment (start 170.8 130.81) (end 170.8 128.285) (width 1) (layer "B.Cu") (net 2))
 (segment (start 114.935 137.16) (end 109.855 132.08) (width 1) (layer "B.Cu") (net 2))
 (segment (start 177.927 103.632) (end 182.88 108.585) (width 1) (layer "B.Cu") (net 2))
 (segment (start 118.364 102.616) (end 138.176 102.616) (width 1) (layer "B.Cu") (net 2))
 (segment (start 144.78 112.268) (end 143.256 110.744) (width 1) (layer "B.Cu") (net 2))
 (segment (start 162.56 114.3) (end 162.56 116.84) (width 1) (layer "B.Cu") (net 2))
 (segment (start 165.1 124.46) (end 165.1 121.92) (width 1) (layer "B.Cu") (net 2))
 (segment (start 165.1 121.92) (end 165.1 121.285) (width 1) (layer "B.Cu") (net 2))
 (segment (start 135.255 106.045) (end 123.825 106.045) (width 1) (layer "B.Cu") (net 2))
 (segment (start 182.88 108.585) (end 182.88 127.635) (width 1) (layer "B.Cu") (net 2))
 (segment (start 123.825 106.045) (end 123.175 106.695) (width 1) (layer "B.Cu") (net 2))
 (segment (start 165.1 116.84) (end 163.83 118.11) (width 1) (layer "B.Cu") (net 2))
 (segment (start 160.528 112.268) (end 144.78 112.268) (width 1) (layer "B.Cu") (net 2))
 (segment (start 143.256 110.744) (end 143.256 106.68) (width 1) (layer "B.Cu") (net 2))
 (segment (start 135.88 106.67) (end 135.255 106.045) (width 1) (layer "B.Cu") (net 2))
 (segment (start 153.3525 133.6675) (end 149.86 137.16) (width 1) (layer "B.Cu") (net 2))
 (segment (start 165.1 121.285) (end 163.83 120.015) (width 1) (layer "B.Cu") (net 2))
 (segment (start 165.1 114.3) (end 165.1 116.84) (width 1) (layer "B.Cu") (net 2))
 (segment (start 162.56 121.285) (end 162.56 121.92) (width 1) (layer "B.Cu") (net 2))
 (segment (start 135.88 111.516) (end 135.88 106.67) (width 1) (layer "B.Cu") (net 2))
 (segment (start 140.208 104.648) (end 140.208 109.728) (width 1) (layer "B.Cu") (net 2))
 (segment (start 168.26 133.35) (end 167.64 133.35) (width 1) (layer "B.Cu") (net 2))
 (segment (start 177.165 133.35) (end 167.64 133.35) (width 1) (layer "B.Cu") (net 2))
 (segment (start 123.18 108.405) (end 123.175 108.4) (width 1) (layer "B.Cu") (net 2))
 (segment (start 146.304 103.632) (end 177.927 103.632) (width 1) (layer "B.Cu") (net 2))
 (segment (start 109.855 111.125) (end 118.364 102.616) (width 1) (layer "B.Cu") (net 2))
 (segment (start 135.88 114.3) (end 135.88 111.516) (width 1) (layer "B.Cu") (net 2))
 (segment (start 170.8 130.81) (end 168.26 133.35) (width 1) (layer "B.Cu") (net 2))
 (segment (start 162.56 114.3) (end 160.528 112.268) (width 1) (layer "B.Cu") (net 2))
 (segment (start 123.175 106.695) (end 123.175 108.4) (width 1) (layer "B.Cu") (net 2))
 (segment (start 182.88 127.635) (end 177.165 133.35) (width 1) (layer "B.Cu") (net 2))
 (segment (start 130.81 134.62) (end 134.62 134.62) (width 1) (layer "B.Cu") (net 4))
 (segment (start 118.11 121.92) (end 130.81 134.62) (width 1) (layer "B.Cu") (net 4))
 (segment (start 134.62 134.62) (end 147.32 134.62) (width 1) (layer "B.Cu") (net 4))
 (segment (start 118.1 121.92) (end 118.11 121.92) (width 1) (layer "B.Cu") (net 4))
 (segment (start 147.32 134.62) (end 157.48 124.46) (width 1) (layer "B.Cu") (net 4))
 (segment (start 144.78 132.08) (end 134.62 132.08) (width 1) (layer "B.Cu") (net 7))
 (segment (start 152.4 124.46) (end 144.78 132.08) (width 1) (layer "B.Cu") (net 7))
 (segment (start 134.62 132.08) (end 130.8 132.08) (width 1) (layer "B.Cu") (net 7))
 (segment (start 130.8 132.08) (end 120.64 121.92) (width 1) (layer "B.Cu") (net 7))
 (segment (start 123.18 121.92) (end 130.8 129.54) (width 1) (layer "B.Cu") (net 6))
 (segment (start 130.8 129.54) (end 134.62 129.54) (width 1) (layer "B.Cu") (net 6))
 (segment (start 142.24 129.54) (end 147.32 124.46) (width 1) (layer "B.Cu") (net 6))
 (segment (start 134.62 129.54) (end 142.24 129.54) (width 1) (layer "B.Cu") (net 6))
 (segment (start 125.72 121.92) (end 130.8 127) (width 1) (layer "B.Cu") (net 3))
 (segment (start 130.8 127) (end 134.62 127) (width 1) (layer "B.Cu") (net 3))
 (segment (start 142.24 124.46) (end 139.7 127) (width 1) (layer "B.Cu") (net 3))
 (segment (start 139.7 127) (end 134.62 127) (width 1) (layer "B.Cu") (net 3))
 (segment (start 128.26 120.66) (end 128.27 120.65) (width 1) (layer "B.Cu") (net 8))
 (segment (start 115.57 127) (end 118.11 129.54) (width 1) (layer "B.Cu") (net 8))
 (segment (start 115.57 120.65) (end 115.57 127) (width 1) (layer "B.Cu") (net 8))
 (segment (start 116.205 120.015) (end 115.57 120.65) (width 1) (layer "B.Cu") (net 8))
 (segment (start 128.26 121.92) (end 128.26 120.66) (width 1) (layer "B.Cu") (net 8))
 (segment (start 127.635 120.015) (end 116.205 120.015) (width 1) (layer "B.Cu") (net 8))
 (segment (start 128.27 120.65) (end 127.635 120.015) (width 1) (layer "B.Cu") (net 8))
 (segment (start 130.8 119.39) (end 130.81 119.38) (width 1) (layer "B.Cu") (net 9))
 (segment (start 129.54 118.11) (end 114.935 118.11) (width 1) (layer "B.Cu") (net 9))
 (segment (start 113.665 128.905) (end 116.84 132.08) (width 1) (layer "B.Cu") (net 9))
 (segment (start 113.665 119.38) (end 113.665 128.905) (width 1) (layer "B.Cu") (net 9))
 (segment (start 114.935 118.11) (end 113.665 119.38) (width 1) (layer "B.Cu") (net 9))
 (segment (start 130.81 119.38) (end 129.54 118.11) (width 1) (layer "B.Cu") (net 9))
 (segment (start 130.8 121.92) (end 130.8 119.39) (width 1) (layer "B.Cu") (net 9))
 (segment (start 116.84 132.08) (end 118.11 132.08) (width 1) (layer "B.Cu") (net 9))
 (segment (start 173.355 125.73) (end 173.355 128.27) (width 1) (layer "B.Cu") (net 19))
 (segment (start 173.355 128.27) (end 173.355 130.795) (width 1) (layer "B.Cu") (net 19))
 (segment (start 175.895 123.19) (end 175.895 119.38) (width 1) (layer "B.Cu") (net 19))
 (segment (start 173.355 125.73) (end 175.895 123.19) (width 1) (layer "B.Cu") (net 19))
 (segment (start 173.355 130.795) (end 173.34 130.81) (width 1) (layer "B.Cu") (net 19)))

